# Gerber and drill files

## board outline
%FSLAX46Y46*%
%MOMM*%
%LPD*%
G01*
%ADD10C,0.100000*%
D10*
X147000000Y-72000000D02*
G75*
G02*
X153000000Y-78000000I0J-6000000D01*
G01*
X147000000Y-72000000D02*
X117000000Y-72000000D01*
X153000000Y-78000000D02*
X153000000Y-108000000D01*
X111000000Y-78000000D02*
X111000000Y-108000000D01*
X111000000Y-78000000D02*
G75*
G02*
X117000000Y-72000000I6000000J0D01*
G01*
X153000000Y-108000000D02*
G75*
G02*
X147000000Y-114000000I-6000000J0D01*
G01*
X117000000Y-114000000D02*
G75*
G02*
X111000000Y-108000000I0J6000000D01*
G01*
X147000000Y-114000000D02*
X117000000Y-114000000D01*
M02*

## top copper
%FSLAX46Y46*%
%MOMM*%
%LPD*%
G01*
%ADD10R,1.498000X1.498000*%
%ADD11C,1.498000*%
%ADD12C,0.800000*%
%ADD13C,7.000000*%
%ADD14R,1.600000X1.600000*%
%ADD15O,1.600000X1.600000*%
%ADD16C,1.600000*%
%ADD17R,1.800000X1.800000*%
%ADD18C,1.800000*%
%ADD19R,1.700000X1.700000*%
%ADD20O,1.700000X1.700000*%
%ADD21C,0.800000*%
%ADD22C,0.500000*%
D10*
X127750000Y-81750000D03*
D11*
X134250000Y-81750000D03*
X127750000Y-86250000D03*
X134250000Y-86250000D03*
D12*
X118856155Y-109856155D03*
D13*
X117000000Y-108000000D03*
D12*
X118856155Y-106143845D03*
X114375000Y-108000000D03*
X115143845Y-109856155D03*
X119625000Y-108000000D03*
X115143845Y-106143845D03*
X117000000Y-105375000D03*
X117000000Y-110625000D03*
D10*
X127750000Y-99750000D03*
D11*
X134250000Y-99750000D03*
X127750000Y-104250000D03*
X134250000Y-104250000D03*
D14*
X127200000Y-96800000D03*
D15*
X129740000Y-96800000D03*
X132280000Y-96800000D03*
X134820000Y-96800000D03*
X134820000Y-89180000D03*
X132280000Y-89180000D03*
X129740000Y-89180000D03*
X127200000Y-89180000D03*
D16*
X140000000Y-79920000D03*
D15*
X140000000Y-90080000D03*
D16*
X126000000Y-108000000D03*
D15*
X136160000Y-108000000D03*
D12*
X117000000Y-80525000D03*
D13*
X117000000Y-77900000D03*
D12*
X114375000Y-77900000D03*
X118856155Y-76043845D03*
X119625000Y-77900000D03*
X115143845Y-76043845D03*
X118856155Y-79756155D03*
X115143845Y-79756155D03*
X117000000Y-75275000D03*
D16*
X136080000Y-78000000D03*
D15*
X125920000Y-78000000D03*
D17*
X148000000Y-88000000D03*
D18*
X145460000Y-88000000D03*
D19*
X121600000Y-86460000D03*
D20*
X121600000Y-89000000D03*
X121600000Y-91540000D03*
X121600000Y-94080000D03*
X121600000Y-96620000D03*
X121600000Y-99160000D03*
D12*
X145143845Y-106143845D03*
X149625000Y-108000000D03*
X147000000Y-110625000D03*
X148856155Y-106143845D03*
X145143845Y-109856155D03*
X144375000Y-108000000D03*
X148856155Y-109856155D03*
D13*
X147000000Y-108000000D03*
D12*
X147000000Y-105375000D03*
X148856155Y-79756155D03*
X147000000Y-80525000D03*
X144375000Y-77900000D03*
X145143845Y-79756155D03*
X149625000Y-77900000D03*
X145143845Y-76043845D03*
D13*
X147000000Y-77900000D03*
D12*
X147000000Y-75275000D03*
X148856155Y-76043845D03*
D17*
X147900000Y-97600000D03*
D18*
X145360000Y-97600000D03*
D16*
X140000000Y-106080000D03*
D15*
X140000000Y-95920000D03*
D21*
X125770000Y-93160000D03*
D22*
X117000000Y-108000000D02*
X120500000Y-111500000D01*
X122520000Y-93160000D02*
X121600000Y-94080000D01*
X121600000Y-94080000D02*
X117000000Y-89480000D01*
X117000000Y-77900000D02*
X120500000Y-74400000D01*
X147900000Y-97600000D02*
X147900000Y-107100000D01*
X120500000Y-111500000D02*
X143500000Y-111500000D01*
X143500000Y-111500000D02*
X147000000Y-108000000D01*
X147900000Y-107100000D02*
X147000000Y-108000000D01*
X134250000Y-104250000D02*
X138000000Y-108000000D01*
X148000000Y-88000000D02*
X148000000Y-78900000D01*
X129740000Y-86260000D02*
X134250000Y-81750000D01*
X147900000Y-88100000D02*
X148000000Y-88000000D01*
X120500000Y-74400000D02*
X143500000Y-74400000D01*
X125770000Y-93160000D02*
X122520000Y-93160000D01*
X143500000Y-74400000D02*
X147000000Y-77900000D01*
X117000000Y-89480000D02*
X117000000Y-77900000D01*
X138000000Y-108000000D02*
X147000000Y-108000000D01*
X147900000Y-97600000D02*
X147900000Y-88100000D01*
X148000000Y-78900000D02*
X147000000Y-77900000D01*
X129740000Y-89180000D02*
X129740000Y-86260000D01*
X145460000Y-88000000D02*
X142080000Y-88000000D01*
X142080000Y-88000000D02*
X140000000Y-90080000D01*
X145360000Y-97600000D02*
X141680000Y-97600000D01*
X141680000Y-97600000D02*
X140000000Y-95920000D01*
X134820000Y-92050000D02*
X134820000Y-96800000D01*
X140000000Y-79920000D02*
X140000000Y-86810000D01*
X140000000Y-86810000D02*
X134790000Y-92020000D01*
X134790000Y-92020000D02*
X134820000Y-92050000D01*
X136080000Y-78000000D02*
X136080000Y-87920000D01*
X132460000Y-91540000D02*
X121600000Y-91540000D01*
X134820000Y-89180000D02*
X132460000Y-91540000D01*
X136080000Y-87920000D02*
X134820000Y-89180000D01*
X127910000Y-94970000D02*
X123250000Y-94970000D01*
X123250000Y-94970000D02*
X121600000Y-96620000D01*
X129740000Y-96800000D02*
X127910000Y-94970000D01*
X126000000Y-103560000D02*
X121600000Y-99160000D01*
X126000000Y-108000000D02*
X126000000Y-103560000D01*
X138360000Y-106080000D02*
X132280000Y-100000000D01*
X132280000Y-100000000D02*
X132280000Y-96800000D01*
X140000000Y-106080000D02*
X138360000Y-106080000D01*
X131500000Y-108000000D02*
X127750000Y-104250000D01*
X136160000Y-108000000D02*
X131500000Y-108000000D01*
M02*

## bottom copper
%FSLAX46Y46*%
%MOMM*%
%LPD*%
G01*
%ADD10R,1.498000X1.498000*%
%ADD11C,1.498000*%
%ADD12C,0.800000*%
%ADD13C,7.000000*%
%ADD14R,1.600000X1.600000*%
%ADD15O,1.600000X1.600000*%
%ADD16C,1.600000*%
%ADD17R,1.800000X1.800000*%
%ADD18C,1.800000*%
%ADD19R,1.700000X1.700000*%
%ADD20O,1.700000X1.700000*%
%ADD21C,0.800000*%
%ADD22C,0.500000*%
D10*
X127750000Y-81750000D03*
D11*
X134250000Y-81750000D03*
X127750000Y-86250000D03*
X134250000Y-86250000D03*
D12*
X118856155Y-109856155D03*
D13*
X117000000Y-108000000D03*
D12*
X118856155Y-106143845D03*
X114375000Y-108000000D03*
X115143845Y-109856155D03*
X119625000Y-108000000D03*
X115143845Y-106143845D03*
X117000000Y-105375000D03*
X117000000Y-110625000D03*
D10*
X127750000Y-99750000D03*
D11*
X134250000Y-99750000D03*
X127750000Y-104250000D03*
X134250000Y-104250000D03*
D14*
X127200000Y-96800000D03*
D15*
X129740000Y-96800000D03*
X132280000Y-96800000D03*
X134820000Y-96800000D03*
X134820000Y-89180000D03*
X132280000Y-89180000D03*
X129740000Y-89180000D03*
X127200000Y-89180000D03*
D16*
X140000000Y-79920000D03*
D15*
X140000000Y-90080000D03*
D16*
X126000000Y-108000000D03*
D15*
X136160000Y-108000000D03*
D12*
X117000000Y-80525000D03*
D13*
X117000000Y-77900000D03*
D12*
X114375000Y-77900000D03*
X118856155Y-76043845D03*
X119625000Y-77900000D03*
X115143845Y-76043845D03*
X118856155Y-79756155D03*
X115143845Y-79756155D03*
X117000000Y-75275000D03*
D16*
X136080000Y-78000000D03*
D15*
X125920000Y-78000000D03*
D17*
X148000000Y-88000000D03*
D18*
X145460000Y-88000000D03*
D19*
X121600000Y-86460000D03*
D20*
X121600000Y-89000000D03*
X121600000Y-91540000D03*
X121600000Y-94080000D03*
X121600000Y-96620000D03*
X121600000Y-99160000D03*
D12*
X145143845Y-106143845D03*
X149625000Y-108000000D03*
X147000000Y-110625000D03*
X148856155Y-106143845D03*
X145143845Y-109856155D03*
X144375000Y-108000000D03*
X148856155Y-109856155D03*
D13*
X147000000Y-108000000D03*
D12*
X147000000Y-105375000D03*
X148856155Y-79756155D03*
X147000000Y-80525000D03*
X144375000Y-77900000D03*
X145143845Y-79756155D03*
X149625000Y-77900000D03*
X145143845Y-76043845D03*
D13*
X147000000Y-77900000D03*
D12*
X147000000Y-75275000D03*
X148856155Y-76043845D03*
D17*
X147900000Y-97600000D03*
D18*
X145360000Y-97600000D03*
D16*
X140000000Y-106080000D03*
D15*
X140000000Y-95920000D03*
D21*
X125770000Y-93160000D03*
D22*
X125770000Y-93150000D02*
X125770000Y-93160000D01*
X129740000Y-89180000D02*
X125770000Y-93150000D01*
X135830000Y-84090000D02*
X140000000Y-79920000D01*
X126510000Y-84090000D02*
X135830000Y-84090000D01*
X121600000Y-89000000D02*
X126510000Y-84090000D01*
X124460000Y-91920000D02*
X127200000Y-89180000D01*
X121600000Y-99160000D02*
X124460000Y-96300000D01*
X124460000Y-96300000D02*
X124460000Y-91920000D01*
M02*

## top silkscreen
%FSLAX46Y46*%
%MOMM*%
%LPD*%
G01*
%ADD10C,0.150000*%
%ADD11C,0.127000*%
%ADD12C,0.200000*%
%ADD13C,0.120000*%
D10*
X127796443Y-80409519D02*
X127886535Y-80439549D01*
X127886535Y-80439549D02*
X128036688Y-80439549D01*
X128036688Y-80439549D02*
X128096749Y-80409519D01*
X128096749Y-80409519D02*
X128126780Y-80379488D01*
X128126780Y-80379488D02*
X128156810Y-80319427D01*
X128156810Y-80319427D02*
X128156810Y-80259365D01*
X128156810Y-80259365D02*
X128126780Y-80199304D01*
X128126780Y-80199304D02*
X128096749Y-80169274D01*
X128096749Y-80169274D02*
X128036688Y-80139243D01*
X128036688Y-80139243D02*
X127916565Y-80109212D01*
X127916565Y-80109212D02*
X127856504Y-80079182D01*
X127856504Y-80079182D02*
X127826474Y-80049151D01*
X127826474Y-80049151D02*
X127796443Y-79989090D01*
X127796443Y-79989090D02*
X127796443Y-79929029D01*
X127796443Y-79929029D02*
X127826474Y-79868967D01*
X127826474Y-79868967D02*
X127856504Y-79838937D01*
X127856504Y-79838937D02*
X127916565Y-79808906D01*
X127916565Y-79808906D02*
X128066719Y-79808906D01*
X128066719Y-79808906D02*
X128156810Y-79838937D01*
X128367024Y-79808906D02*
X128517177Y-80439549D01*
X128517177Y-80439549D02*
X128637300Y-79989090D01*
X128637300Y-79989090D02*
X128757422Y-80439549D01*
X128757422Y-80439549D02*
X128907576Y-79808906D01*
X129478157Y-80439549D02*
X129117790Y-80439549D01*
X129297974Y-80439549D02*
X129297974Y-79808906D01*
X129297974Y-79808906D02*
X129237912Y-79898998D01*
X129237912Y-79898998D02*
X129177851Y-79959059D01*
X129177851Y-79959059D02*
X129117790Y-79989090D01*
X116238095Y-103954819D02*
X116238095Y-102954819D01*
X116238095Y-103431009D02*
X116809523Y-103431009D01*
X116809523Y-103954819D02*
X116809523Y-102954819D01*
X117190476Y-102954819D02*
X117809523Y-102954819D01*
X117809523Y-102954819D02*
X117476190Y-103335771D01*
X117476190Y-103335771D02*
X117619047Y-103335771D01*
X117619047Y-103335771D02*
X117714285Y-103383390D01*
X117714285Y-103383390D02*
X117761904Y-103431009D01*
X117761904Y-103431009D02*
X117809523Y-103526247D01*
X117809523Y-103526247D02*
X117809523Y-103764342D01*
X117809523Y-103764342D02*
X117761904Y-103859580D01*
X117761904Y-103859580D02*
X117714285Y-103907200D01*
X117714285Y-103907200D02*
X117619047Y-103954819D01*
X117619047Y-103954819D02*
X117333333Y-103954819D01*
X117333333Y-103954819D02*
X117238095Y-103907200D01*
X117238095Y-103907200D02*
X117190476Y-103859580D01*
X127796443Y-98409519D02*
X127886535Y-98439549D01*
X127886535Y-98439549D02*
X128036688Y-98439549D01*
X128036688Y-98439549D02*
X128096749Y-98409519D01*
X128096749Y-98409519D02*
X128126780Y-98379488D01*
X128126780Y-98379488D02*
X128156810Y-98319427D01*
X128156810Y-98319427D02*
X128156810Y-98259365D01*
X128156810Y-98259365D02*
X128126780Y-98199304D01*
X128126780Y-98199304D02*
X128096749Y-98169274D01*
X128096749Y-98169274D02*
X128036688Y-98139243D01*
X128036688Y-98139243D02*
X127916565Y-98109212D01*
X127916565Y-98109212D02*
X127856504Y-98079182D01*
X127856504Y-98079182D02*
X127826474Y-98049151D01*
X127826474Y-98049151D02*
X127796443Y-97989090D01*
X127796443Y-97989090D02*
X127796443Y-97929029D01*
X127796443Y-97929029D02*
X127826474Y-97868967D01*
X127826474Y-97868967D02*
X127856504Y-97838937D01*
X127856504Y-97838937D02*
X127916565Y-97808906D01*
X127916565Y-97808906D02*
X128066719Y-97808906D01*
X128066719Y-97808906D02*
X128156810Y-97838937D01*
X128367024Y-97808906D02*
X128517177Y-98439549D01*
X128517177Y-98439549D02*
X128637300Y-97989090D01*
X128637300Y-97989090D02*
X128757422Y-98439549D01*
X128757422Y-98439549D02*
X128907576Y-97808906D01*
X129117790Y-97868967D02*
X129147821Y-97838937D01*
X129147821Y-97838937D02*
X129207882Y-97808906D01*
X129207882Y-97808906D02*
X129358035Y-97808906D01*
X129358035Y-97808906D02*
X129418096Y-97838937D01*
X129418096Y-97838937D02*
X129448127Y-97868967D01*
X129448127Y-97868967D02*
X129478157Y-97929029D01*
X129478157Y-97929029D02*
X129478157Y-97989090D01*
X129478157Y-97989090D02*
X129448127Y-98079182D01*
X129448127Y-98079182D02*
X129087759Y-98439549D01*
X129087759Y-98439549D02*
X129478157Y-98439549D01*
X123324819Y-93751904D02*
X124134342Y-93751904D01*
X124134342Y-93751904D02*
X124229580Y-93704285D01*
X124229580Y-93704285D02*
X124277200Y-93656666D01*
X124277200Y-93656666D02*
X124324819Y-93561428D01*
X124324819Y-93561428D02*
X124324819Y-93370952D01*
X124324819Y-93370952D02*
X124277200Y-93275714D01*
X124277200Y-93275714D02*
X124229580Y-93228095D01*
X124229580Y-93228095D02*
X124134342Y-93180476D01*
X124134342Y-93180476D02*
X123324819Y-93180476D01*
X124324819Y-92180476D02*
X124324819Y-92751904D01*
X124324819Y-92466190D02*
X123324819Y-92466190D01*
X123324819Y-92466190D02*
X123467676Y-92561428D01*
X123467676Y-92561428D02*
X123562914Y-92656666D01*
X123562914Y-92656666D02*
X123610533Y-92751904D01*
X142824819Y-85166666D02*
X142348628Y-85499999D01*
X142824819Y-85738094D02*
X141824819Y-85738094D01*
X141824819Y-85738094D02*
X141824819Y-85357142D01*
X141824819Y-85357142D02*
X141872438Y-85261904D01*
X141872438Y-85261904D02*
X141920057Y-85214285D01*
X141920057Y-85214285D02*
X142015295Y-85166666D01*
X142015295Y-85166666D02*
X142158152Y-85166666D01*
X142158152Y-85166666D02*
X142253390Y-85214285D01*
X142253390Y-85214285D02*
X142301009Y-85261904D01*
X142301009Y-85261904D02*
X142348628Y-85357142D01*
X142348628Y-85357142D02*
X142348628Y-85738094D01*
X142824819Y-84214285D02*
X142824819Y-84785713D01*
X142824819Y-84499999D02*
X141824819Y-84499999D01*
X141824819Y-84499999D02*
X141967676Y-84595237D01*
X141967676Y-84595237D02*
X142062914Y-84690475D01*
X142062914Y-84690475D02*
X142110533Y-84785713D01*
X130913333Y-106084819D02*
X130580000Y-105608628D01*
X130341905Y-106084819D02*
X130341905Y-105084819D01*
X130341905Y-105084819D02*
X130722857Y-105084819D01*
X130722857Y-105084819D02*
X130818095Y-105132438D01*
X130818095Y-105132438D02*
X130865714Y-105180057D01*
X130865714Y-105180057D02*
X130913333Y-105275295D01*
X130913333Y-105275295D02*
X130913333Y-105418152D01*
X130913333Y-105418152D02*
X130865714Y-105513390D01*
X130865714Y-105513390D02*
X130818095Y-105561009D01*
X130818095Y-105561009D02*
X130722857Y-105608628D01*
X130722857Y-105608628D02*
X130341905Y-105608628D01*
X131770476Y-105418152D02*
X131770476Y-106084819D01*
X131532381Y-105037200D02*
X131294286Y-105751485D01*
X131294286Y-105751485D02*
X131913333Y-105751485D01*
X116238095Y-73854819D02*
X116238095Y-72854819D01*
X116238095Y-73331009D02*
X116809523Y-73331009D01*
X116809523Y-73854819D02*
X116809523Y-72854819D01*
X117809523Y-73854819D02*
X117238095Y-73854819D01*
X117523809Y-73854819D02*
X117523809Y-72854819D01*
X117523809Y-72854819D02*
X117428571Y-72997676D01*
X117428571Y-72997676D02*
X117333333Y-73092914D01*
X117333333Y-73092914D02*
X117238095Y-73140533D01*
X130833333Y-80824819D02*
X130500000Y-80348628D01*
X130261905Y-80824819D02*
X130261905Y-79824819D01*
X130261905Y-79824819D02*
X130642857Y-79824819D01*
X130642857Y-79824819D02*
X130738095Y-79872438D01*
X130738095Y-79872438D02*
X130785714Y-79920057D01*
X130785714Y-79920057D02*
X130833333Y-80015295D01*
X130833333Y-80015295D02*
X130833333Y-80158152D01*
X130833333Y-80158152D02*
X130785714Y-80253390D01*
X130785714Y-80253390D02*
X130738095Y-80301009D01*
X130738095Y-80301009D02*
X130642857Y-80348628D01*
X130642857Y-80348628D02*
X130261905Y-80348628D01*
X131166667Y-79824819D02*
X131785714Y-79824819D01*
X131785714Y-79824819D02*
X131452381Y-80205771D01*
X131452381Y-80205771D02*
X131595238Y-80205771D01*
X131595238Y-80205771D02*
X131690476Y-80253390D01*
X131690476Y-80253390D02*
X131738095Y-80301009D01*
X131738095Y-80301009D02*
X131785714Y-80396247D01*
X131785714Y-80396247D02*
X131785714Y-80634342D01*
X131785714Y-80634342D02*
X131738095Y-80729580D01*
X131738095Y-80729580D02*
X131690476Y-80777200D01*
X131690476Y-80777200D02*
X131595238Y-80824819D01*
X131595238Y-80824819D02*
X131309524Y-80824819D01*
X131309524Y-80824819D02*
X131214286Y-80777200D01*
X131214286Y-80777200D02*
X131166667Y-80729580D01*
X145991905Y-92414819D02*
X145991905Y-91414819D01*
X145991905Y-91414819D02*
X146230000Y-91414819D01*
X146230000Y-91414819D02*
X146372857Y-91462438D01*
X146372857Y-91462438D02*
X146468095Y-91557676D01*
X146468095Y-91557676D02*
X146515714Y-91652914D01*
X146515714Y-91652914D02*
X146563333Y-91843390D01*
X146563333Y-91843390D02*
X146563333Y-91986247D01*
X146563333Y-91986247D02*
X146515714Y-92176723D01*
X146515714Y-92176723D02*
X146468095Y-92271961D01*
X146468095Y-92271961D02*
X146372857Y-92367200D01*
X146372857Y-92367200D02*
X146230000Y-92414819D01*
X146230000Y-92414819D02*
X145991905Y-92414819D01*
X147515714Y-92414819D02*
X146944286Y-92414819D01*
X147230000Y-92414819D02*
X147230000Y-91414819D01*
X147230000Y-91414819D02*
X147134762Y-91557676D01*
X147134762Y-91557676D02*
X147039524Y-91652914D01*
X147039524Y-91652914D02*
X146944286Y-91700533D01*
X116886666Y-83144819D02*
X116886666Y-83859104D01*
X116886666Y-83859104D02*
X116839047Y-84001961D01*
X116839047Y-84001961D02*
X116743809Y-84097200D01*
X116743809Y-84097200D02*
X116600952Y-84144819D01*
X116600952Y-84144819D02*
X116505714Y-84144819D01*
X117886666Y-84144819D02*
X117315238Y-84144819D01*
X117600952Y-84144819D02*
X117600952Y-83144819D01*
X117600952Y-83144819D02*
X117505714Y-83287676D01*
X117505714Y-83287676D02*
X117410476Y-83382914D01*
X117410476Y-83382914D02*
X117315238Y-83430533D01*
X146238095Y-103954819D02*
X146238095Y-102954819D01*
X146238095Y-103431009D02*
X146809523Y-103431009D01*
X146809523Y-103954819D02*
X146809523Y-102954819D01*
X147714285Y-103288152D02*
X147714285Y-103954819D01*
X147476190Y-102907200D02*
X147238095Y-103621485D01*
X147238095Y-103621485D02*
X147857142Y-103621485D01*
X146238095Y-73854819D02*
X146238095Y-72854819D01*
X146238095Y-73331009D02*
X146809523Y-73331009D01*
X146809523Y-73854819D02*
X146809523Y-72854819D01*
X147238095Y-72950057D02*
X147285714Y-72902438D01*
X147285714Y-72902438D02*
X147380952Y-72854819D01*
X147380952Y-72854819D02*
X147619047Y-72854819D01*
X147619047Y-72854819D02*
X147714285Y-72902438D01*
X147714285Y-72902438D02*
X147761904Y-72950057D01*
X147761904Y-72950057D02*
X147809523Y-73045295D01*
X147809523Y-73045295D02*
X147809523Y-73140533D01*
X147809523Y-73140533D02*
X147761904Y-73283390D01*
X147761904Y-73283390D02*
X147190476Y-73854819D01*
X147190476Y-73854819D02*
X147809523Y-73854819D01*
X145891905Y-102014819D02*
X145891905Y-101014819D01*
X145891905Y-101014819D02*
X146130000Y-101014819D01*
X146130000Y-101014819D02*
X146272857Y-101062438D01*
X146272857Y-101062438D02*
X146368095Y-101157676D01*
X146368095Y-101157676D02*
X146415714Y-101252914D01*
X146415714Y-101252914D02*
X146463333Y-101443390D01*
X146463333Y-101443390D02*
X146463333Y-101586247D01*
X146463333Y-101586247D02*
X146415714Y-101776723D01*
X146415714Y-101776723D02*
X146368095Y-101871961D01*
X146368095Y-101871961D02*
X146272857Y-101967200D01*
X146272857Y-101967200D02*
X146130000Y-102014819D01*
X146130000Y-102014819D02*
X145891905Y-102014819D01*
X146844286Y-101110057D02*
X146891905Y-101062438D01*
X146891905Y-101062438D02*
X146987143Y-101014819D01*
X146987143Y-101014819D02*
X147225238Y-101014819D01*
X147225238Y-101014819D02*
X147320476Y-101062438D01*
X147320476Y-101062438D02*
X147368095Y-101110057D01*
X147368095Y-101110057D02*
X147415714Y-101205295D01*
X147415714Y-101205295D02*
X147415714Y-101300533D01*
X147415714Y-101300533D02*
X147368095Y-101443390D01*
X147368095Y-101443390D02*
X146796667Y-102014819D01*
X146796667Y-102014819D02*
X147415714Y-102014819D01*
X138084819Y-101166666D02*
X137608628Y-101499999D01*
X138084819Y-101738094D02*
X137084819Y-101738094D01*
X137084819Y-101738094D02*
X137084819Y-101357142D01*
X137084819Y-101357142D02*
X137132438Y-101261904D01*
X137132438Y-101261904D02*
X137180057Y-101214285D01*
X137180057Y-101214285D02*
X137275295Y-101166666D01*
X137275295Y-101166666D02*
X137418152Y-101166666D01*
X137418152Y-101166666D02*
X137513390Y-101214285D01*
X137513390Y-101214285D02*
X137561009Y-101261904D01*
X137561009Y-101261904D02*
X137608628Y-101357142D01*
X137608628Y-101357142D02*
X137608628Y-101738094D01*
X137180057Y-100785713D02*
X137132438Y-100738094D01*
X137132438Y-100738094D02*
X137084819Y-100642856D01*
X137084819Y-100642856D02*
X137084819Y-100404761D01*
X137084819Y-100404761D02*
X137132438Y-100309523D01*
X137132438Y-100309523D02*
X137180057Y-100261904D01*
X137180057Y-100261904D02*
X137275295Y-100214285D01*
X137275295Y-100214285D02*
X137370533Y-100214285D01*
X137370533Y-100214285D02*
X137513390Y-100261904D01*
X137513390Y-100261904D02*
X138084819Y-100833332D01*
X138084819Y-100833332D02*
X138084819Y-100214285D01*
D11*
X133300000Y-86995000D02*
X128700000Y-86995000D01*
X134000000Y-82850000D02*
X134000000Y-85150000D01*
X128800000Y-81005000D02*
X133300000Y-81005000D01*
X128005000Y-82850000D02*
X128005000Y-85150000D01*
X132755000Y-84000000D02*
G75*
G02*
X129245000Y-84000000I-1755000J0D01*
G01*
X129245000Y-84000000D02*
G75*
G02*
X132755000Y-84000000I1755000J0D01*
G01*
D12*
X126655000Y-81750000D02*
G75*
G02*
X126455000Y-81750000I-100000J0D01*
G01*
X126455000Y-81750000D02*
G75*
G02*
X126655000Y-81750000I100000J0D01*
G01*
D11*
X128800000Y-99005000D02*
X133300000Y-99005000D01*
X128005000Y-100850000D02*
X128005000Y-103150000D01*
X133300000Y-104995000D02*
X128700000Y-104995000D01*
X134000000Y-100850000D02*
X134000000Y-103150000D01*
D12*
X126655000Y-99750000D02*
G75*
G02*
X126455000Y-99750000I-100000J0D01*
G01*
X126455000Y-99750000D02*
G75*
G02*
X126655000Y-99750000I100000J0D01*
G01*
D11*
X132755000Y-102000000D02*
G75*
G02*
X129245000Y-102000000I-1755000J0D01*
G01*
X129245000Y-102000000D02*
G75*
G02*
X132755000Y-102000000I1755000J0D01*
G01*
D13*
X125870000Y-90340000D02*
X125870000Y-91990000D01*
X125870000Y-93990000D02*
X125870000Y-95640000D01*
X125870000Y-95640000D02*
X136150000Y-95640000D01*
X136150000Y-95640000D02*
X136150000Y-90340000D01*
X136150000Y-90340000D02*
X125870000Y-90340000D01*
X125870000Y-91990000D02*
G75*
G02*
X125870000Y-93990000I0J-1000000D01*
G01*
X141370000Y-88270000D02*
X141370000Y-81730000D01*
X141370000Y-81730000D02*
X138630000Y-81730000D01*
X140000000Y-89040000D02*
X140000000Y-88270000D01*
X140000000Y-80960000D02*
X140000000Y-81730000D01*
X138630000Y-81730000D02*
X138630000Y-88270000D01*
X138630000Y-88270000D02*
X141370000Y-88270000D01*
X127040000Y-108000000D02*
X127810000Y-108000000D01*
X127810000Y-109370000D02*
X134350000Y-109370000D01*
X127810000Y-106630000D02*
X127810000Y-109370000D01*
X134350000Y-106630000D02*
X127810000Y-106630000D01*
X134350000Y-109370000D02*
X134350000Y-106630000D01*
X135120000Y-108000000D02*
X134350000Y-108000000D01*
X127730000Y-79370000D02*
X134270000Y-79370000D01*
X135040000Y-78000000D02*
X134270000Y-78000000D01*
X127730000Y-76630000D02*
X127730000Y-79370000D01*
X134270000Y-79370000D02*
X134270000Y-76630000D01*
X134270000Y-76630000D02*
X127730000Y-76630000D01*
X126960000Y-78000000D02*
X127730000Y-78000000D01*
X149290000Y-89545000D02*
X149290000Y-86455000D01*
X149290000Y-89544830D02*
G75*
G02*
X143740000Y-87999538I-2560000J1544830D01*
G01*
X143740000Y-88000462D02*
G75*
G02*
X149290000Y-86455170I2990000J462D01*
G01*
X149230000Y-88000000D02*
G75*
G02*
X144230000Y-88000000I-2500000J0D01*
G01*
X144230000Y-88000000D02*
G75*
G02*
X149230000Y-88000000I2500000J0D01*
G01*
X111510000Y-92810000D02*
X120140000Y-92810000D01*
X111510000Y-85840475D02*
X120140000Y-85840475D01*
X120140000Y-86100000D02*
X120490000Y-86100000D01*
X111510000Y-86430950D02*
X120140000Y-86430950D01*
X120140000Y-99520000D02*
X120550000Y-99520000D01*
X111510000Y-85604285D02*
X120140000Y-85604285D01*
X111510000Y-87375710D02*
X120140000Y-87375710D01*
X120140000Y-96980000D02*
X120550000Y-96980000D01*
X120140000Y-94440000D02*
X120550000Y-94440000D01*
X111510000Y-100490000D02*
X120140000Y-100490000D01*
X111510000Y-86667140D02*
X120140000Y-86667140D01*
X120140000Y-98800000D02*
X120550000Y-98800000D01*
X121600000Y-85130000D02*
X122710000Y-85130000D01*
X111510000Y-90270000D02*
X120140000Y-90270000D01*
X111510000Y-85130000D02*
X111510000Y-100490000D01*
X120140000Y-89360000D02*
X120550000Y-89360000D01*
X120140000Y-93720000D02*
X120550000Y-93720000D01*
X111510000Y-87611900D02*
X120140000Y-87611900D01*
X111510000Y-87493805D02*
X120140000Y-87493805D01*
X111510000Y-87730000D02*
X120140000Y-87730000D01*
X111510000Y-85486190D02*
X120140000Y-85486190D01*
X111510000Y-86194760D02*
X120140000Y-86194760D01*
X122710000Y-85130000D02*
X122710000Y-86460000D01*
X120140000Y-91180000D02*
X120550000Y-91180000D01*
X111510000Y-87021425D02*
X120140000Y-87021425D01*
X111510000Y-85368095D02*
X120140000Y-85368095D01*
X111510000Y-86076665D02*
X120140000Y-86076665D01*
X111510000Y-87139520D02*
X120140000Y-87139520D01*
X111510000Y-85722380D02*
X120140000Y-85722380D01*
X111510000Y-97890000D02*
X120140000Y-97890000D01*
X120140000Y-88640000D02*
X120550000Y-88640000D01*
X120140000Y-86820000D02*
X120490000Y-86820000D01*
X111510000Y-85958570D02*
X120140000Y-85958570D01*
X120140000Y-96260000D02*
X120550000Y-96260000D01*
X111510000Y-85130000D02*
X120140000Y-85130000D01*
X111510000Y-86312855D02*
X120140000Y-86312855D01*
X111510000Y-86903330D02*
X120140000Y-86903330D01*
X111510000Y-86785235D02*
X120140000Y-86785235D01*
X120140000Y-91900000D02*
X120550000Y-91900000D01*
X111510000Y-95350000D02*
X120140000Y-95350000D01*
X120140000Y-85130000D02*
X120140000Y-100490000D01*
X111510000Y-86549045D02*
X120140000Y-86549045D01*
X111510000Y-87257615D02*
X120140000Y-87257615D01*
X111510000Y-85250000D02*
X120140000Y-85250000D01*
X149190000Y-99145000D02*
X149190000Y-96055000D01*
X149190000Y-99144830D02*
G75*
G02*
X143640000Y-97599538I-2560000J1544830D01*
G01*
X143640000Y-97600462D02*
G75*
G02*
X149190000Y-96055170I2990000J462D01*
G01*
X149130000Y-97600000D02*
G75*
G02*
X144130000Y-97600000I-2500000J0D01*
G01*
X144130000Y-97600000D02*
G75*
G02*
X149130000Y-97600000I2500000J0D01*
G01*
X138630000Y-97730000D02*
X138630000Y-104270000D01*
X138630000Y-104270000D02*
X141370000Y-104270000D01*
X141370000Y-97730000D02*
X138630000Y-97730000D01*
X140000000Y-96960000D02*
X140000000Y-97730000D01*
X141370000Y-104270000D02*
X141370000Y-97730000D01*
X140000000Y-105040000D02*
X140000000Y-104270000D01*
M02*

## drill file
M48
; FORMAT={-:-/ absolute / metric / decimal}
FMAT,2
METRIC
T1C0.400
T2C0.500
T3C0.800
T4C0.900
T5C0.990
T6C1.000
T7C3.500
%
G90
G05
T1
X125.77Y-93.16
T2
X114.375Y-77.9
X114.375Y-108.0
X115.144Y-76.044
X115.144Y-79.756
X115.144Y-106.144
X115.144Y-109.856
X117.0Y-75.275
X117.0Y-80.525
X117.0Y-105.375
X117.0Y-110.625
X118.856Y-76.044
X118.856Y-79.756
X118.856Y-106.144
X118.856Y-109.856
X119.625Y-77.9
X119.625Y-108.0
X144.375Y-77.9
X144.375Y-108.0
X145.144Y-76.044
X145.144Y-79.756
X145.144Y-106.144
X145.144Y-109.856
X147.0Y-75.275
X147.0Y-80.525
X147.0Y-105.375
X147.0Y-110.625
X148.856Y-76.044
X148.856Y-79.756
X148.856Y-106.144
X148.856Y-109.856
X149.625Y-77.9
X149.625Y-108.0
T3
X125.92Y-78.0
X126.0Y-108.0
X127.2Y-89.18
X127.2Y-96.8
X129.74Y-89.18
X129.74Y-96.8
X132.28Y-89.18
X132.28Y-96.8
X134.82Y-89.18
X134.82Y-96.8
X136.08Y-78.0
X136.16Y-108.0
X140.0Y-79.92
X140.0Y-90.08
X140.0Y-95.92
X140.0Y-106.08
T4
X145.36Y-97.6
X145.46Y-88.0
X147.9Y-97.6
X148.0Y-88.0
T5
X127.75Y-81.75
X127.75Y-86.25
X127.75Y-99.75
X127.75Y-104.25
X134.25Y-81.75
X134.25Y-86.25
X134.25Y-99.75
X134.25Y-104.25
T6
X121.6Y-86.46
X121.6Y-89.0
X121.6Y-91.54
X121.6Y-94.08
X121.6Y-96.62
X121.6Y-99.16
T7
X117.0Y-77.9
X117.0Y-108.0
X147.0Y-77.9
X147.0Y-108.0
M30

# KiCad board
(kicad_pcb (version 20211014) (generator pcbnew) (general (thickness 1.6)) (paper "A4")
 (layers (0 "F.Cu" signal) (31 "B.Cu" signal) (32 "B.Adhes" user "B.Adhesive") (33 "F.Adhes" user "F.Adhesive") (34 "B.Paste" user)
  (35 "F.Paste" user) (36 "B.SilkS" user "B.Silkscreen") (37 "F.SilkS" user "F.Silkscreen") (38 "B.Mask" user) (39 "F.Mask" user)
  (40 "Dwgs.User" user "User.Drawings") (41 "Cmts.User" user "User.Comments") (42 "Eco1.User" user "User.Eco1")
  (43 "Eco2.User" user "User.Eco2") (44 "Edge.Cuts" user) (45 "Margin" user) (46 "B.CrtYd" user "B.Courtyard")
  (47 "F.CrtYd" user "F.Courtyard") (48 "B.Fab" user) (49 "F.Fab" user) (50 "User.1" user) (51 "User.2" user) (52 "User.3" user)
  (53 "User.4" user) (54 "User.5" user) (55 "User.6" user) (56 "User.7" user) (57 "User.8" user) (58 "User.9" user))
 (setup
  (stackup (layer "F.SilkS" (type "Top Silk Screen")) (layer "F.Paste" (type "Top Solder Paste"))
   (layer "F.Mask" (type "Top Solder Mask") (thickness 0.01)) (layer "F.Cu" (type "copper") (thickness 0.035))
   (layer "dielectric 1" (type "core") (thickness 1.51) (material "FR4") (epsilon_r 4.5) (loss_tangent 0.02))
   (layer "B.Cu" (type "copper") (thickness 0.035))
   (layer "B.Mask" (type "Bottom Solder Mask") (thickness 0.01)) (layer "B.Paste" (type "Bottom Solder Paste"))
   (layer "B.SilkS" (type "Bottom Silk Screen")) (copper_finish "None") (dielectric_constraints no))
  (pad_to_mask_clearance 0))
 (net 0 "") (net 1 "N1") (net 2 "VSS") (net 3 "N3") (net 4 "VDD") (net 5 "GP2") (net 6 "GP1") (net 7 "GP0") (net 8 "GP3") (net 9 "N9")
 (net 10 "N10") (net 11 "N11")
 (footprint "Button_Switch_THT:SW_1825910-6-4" (layer "F.Cu") (at 131 84)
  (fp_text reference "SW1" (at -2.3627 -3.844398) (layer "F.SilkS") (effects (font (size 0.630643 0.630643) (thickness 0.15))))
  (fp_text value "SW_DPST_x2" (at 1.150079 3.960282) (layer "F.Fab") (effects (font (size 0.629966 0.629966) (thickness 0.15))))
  (fp_line (start 2.3 2.995) (end -2.3 2.995) (layer "F.SilkS") (width 0.127))
  (fp_line (start 3 -1.15) (end 3 1.15) (layer "F.SilkS") (width 0.127))
  (fp_line (start -2.2 -2.995) (end 2.3 -2.995) (layer "F.SilkS") (width 0.127))
  (fp_line (start -2.995 -1.15) (end -2.995 1.15) (layer "F.SilkS") (width 0.127))
  (fp_circle (center 0 0) (end 1.755 0) (layer "F.SilkS") (width 0.127) (fill none))
  (fp_circle (center -4.445 -2.25) (end -4.345 -2.25) (layer "F.SilkS") (width 0.2) (fill none))
  (pad "1" thru_hole rect locked (at -3.25 -2.25) (size 1.498 1.498) (drill 0.99) (layers *.Cu *.Mask) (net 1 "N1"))
  (pad "2" thru_hole circle locked (at 3.25 -2.25) (size 1.498 1.498) (drill 0.99) (layers *.Cu *.Mask) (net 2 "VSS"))
  (pad "3" thru_hole circle locked (at -3.25 2.25) (size 1.498 1.498) (drill 0.99) (layers *.Cu *.Mask))
  (pad "4" thru_hole circle locked (at 3.25 2.25) (size 1.498 1.498) (drill 0.99) (layers *.Cu *.Mask)))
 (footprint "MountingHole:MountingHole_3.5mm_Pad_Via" (layer "F.Cu") (at 117 108)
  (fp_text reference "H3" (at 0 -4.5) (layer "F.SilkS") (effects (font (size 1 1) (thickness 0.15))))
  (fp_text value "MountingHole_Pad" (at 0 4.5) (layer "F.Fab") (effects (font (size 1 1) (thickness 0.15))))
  (pad "1" thru_hole circle (at 1.856155 1.856155) (size 0.8 0.8) (drill 0.5) (layers *.Cu *.Mask) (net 2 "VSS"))
  (pad "1" thru_hole circle (at 0 0) (size 7 7) (drill 3.5) (layers *.Cu *.Mask) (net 2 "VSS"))
  (pad "1" thru_hole circle (at 1.856155 -1.856155) (size 0.8 0.8) (drill 0.5) (layers *.Cu *.Mask) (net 2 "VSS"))
  (pad "1" thru_hole circle (at -2.625 0) (size 0.8 0.8) (drill 0.5) (layers *.Cu *.Mask) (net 2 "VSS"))
  (pad "1" thru_hole circle (at -1.856155 1.856155) (size 0.8 0.8) (drill 0.5) (layers *.Cu *.Mask) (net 2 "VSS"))
  (pad "1" thru_hole circle (at 2.625 0) (size 0.8 0.8) (drill 0.5) (layers *.Cu *.Mask) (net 2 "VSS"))
  (pad "1" thru_hole circle (at -1.856155 -1.856155) (size 0.8 0.8) (drill 0.5) (layers *.Cu *.Mask) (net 2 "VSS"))
  (pad "1" thru_hole circle (at 0 -2.625) (size 0.8 0.8) (drill 0.5) (layers *.Cu *.Mask) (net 2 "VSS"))
  (pad "1" thru_hole circle (at 0 2.625) (size 0.8 0.8) (drill 0.5) (layers *.Cu *.Mask) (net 2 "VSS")))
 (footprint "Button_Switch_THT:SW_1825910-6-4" (layer "F.Cu") (at 131 102)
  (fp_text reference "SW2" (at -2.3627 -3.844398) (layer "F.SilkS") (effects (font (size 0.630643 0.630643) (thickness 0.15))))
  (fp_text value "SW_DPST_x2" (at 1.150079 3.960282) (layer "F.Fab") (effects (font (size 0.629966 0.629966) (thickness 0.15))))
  (fp_line (start -2.2 -2.995) (end 2.3 -2.995) (layer "F.SilkS") (width 0.127))
  (fp_line (start -2.995 -1.15) (end -2.995 1.15) (layer "F.SilkS") (width 0.127))
  (fp_line (start 2.3 2.995) (end -2.3 2.995) (layer "F.SilkS") (width 0.127))
  (fp_line (start 3 -1.15) (end 3 1.15) (layer "F.SilkS") (width 0.127))
  (fp_circle (center -4.445 -2.25) (end -4.345 -2.25) (layer "F.SilkS") (width 0.2) (fill none))
  (fp_circle (center 0 0) (end 1.755 0) (layer "F.SilkS") (width 0.127) (fill none))
  (pad "1" thru_hole rect locked (at -3.25 -2.25) (size 1.498 1.498) (drill 0.99) (layers *.Cu *.Mask))
  (pad "2" thru_hole circle locked (at 3.25 -2.25) (size 1.498 1.498) (drill 0.99) (layers *.Cu *.Mask))
  (pad "3" thru_hole circle locked (at -3.25 2.25) (size 1.498 1.498) (drill 0.99) (layers *.Cu *.Mask) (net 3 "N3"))
  (pad "4" thru_hole circle locked (at 3.25 2.25) (size 1.498 1.498) (drill 0.99) (layers *.Cu *.Mask) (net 2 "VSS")))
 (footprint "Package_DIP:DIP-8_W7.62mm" (layer "F.Cu") (at 127.2 96.8 90)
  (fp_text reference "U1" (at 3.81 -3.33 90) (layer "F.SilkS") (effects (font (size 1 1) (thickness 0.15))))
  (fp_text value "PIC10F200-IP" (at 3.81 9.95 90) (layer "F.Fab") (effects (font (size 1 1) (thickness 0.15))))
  (fp_line (start 6.46 -1.33) (end 4.81 -1.33) (layer "F.SilkS") (width 0.12))
  (fp_line (start 2.81 -1.33) (end 1.16 -1.33) (layer "F.SilkS") (width 0.12))
  (fp_line (start 1.16 -1.33) (end 1.16 8.95) (layer "F.SilkS") (width 0.12))
  (fp_line (start 1.16 8.95) (end 6.46 8.95) (layer "F.SilkS") (width 0.12))
  (fp_line (start 6.46 8.95) (end 6.46 -1.33) (layer "F.SilkS") (width 0.12))
  (fp_arc (start 4.81 -1.33) (mid 3.81 -0.33) (end 2.81 -1.33) (layer "F.SilkS") (width 0.12))
  (pad "1" thru_hole rect (at 0 0 90) (size 1.6 1.6) (drill 0.8) (layers *.Cu *.Mask))
  (pad "2" thru_hole oval (at 0 2.54 90) (size 1.6 1.6) (drill 0.8) (layers *.Cu *.Mask) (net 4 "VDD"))
  (pad "3" thru_hole oval (at 0 5.08 90) (size 1.6 1.6) (drill 0.8) (layers *.Cu *.Mask) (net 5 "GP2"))
  (pad "4" thru_hole oval (at 0 7.62 90) (size 1.6 1.6) (drill 0.8) (layers *.Cu *.Mask) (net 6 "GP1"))
  (pad "5" thru_hole oval (at 7.62 7.62 90) (size 1.6 1.6) (drill 0.8) (layers *.Cu *.Mask) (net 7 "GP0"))
  (pad "6" thru_hole oval (at 7.62 5.08 90) (size 1.6 1.6) (drill 0.8) (layers *.Cu *.Mask))
  (pad "7" thru_hole oval (at 7.62 2.54 90) (size 1.6 1.6) (drill 0.8) (layers *.Cu *.Mask) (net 2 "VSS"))
  (pad "8" thru_hole oval (at 7.62 0 90) (size 1.6 1.6) (drill 0.8) (layers *.Cu *.Mask) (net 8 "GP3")))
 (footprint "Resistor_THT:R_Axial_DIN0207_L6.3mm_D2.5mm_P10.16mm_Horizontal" (layer "F.Cu") (at 140 79.92 -90)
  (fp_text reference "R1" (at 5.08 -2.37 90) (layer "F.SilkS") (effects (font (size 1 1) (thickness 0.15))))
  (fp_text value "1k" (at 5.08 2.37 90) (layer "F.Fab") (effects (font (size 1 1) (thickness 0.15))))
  (fp_line (start 8.35 -1.37) (end 1.81 -1.37) (layer "F.SilkS") (width 0.12))
  (fp_line (start 1.81 -1.37) (end 1.81 1.37) (layer "F.SilkS") (width 0.12))
  (fp_line (start 9.12 0) (end 8.35 0) (layer "F.SilkS") (width 0.12))
  (fp_line (start 1.04 0) (end 1.81 0) (layer "F.SilkS") (width 0.12))
  (fp_line (start 1.81 1.37) (end 8.35 1.37) (layer "F.SilkS") (width 0.12))
  (fp_line (start 8.35 1.37) (end 8.35 -1.37) (layer "F.SilkS") (width 0.12))
  (pad "1" thru_hole circle (at 0 0 270) (size 1.6 1.6) (drill 0.8) (layers *.Cu *.Mask) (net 6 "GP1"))
  (pad "2" thru_hole oval (at 10.16 0 270) (size 1.6 1.6) (drill 0.8) (layers *.Cu *.Mask) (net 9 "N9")))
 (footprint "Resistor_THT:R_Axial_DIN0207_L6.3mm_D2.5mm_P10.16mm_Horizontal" (layer "F.Cu") (at 126 108)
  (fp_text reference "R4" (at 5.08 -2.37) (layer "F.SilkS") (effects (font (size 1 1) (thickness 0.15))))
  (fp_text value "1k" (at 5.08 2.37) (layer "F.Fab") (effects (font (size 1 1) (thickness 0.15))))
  (fp_line (start 1.04 0) (end 1.81 0) (layer "F.SilkS") (width 0.12))
  (fp_line (start 1.81 1.37) (end 8.35 1.37) (layer "F.SilkS") (width 0.12))
  (fp_line (start 1.81 -1.37) (end 1.81 1.37) (layer "F.SilkS") (width 0.12))
  (fp_line (start 8.35 -1.37) (end 1.81 -1.37) (layer "F.SilkS") (width 0.12))
  (fp_line (start 8.35 1.37) (end 8.35 -1.37) (layer "F.SilkS") (width 0.12))
  (fp_line (start 9.12 0) (end 8.35 0) (layer "F.SilkS") (width 0.12))
  (pad "1" thru_hole circle (at 0 0) (size 1.6 1.6) (drill 0.8) (layers *.Cu *.Mask) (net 8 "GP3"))
  (pad "2" thru_hole oval (at 10.16 0) (size 1.6 1.6) (drill 0.8) (layers *.Cu *.Mask) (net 3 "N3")))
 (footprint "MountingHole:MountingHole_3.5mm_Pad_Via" (layer "F.Cu") (at 117 77.9)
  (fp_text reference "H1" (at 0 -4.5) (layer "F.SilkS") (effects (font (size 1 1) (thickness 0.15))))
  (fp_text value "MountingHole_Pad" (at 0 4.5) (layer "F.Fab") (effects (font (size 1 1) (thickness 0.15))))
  (pad "1" thru_hole circle (at 0 2.625) (size 0.8 0.8) (drill 0.5) (layers *.Cu *.Mask) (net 2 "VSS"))
  (pad "1" thru_hole circle (at 0 0) (size 7 7) (drill 3.5) (layers *.Cu *.Mask) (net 2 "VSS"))
  (pad "1" thru_hole circle (at -2.625 0) (size 0.8 0.8) (drill 0.5) (layers *.Cu *.Mask) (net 2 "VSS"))
  (pad "1" thru_hole circle (at 1.856155 -1.856155) (size 0.8 0.8) (drill 0.5) (layers *.Cu *.Mask) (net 2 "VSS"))
  (pad "1" thru_hole circle (at 2.625 0) (size 0.8 0.8) (drill 0.5) (layers *.Cu *.Mask) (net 2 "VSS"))
  (pad "1" thru_hole circle (at -1.856155 -1.856155) (size 0.8 0.8) (drill 0.5) (layers *.Cu *.Mask) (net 2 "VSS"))
  (pad "1" thru_hole circle (at 1.856155 1.856155) (size 0.8 0.8) (drill 0.5) (layers *.Cu *.Mask) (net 2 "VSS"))
  (pad "1" thru_hole circle (at -1.856155 1.856155) (size 0.8 0.8) (drill 0.5) (layers *.Cu *.Mask) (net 2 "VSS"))
  (pad "1" thru_hole circle (at 0 -2.625) (size 0.8 0.8) (drill 0.5) (layers *.Cu *.Mask) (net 2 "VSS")))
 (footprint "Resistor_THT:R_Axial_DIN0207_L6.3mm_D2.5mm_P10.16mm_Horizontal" (layer "F.Cu") (at 136.08 78 180)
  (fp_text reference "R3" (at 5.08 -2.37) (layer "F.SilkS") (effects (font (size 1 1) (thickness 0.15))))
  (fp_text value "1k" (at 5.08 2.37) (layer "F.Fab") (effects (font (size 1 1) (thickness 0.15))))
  (fp_line (start 8.35 -1.37) (end 1.81 -1.37) (layer "F.SilkS") (width 0.12))
  (fp_line (start 1.04 0) (end 1.81 0) (layer "F.SilkS") (width 0.12))
  (fp_line (start 8.35 1.37) (end 8.35 -1.37) (layer "F.SilkS") (width 0.12))
  (fp_line (start 1.81 -1.37) (end 1.81 1.37) (layer "F.SilkS") (width 0.12))
  (fp_line (start 1.81 1.37) (end 8.35 1.37) (layer "F.SilkS") (width 0.12))
  (fp_line (start 9.12 0) (end 8.35 0) (layer "F.SilkS") (width 0.12))
  (pad "1" thru_hole circle (at 0 0 180) (size 1.6 1.6) (drill 0.8) (layers *.Cu *.Mask) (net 7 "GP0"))
  (pad "2" thru_hole oval (at 10.16 0 180) (size 1.6 1.6) (drill 0.8) (layers *.Cu *.Mask) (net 1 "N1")))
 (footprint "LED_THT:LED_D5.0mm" (layer "F.Cu") (at 148 88 180)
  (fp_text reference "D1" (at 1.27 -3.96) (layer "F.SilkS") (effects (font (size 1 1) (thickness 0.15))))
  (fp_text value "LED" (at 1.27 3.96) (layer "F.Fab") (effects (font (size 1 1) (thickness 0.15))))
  (fp_line (start -1.29 -1.545) (end -1.29 1.545) (layer "F.SilkS") (width 0.12))
  (fp_arc (start -1.29 -1.54483) (mid 2.072002 -2.880433) (end 4.26 0.000462) (layer "F.SilkS") (width 0.12))
  (fp_arc (start 4.26 -0.000462) (mid 2.072002 2.880433) (end -1.29 1.54483) (layer "F.SilkS") (width 0.12))
  (fp_circle (center 1.27 0) (end 3.77 0) (layer "F.SilkS") (width 0.12) (fill none))
  (pad "1" thru_hole rect (at 0 0 180) (size 1.8 1.8) (drill 0.9) (layers *.Cu *.Mask) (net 2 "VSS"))
  (pad "2" thru_hole circle (at 2.54 0 180) (size 1.8 1.8) (drill 0.9) (layers *.Cu *.Mask) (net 9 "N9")))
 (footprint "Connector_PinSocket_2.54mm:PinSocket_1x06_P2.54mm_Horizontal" (layer "F.Cu") (at 121.6 86.46)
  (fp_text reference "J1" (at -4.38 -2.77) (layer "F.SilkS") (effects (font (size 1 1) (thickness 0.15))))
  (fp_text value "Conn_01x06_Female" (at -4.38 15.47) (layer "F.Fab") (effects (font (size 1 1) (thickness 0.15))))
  (fp_line (start -10.09 6.35) (end -1.46 6.35) (layer "F.SilkS") (width 0.12))
  (fp_line (start -10.09 -0.619525) (end -1.46 -0.619525) (layer "F.SilkS") (width 0.12))
  (fp_line (start -1.46 -0.36) (end -1.11 -0.36) (layer "F.SilkS") (width 0.12))
  (fp_line (start -10.09 -0.02905) (end -1.46 -0.02905) (layer "F.SilkS") (width 0.12))
  (fp_line (start -1.46 13.06) (end -1.05 13.06) (layer "F.SilkS") (width 0.12))
  (fp_line (start -10.09 -0.855715) (end -1.46 -0.855715) (layer "F.SilkS") (width 0.12))
  (fp_line (start -10.09 0.91571) (end -1.46 0.91571) (layer "F.SilkS") (width 0.12))
  (fp_line (start -1.46 10.52) (end -1.05 10.52) (layer "F.SilkS") (width 0.12))
  (fp_line (start -1.46 7.98) (end -1.05 7.98) (layer "F.SilkS") (width 0.12))
  (fp_line (start -10.09 14.03) (end -1.46 14.03) (layer "F.SilkS") (width 0.12))
  (fp_line (start -10.09 0.20714) (end -1.46 0.20714) (layer "F.SilkS") (width 0.12))
  (fp_line (start -1.46 12.34) (end -1.05 12.34) (layer "F.SilkS") (width 0.12))
  (fp_line (start 0 -1.33) (end 1.11 -1.33) (layer "F.SilkS") (width 0.12))
  (fp_line (start -10.09 3.81) (end -1.46 3.81) (layer "F.SilkS") (width 0.12))
  (fp_line (start -10.09 -1.33) (end -10.09 14.03) (layer "F.SilkS") (width 0.12))
  (fp_line (start -1.46 2.9) (end -1.05 2.9) (layer "F.SilkS") (width 0.12))
  (fp_line (start -1.46 7.26) (end -1.05 7.26) (layer "F.SilkS") (width 0.12))
  (fp_line (start -10.09 1.1519) (end -1.46 1.1519) (layer "F.SilkS") (width 0.12))
  (fp_line (start -10.09 1.033805) (end -1.46 1.033805) (layer "F.SilkS") (width 0.12))
  (fp_line (start -10.09 1.27) (end -1.46 1.27) (layer "F.SilkS") (width 0.12))
  (fp_line (start -10.09 -0.97381) (end -1.46 -0.97381) (layer "F.SilkS") (width 0.12))
  (fp_line (start -10.09 -0.26524) (end -1.46 -0.26524) (layer "F.SilkS") (width 0.12))
  (fp_line (start 1.11 -1.33) (end 1.11 0) (layer "F.SilkS") (width 0.12))
  (fp_line (start -1.46 4.72) (end -1.05 4.72) (layer "F.SilkS") (width 0.12))
  (fp_line (start -10.09 0.561425) (end -1.46 0.561425) (layer "F.SilkS") (width 0.12))
  (fp_line (start -10.09 -1.091905) (end -1.46 -1.091905) (layer "F.SilkS") (width 0.12))
  (fp_line (start -10.09 -0.383335) (end -1.46 -0.383335) (layer "F.SilkS") (width 0.12))
  (fp_line (start -10.09 0.67952) (end -1.46 0.67952) (layer "F.SilkS") (width 0.12))
  (fp_line (start -10.09 -0.73762) (end -1.46 -0.73762) (layer "F.SilkS") (width 0.12))
  (fp_line (start -10.09 11.43) (end -1.46 11.43) (layer "F.SilkS") (width 0.12))
  (fp_line (start -1.46 2.18) (end -1.05 2.18) (layer "F.SilkS") (width 0.12))
  (fp_line (start -1.46 0.36) (end -1.11 0.36) (layer "F.SilkS") (width 0.12))
  (fp_line (start -10.09 -0.50143) (end -1.46 -0.50143) (layer "F.SilkS") (width 0.12))
  (fp_line (start -1.46 9.8) (end -1.05 9.8) (layer "F.SilkS") (width 0.12))
  (fp_line (start -10.09 -1.33) (end -1.46 -1.33) (layer "F.SilkS") (width 0.12))
  (fp_line (start -10.09 -0.147145) (end -1.46 -0.147145) (layer "F.SilkS") (width 0.12))
  (fp_line (start -10.09 0.44333) (end -1.46 0.44333) (layer "F.SilkS") (width 0.12))
  (fp_line (start -10.09 0.325235) (end -1.46 0.325235) (layer "F.SilkS") (width 0.12))
  (fp_line (start -1.46 5.44) (end -1.05 5.44) (layer "F.SilkS") (width 0.12))
  (fp_line (start -10.09 8.89) (end -1.46 8.89) (layer "F.SilkS") (width 0.12))
  (fp_line (start -1.46 -1.33) (end -1.46 14.03) (layer "F.SilkS") (width 0.12))
  (fp_line (start -10.09 0.089045) (end -1.46 0.089045) (layer "F.SilkS") (width 0.12))
  (fp_line (start -10.09 0.797615) (end -1.46 0.797615) (layer "F.SilkS") (width 0.12))
  (fp_line (start -10.09 -1.21) (end -1.46 -1.21) (layer "F.SilkS") (width 0.12))
  (pad "1" thru_hole rect (at 0 0) (size 1.7 1.7) (drill 1) (layers *.Cu *.Mask) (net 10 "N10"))
  (pad "2" thru_hole oval (at 0 2.54) (size 1.7 1.7) (drill 1) (layers *.Cu *.Mask) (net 6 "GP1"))
  (pad "3" thru_hole oval (at 0 5.08) (size 1.7 1.7) (drill 1) (layers *.Cu *.Mask) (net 7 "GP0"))
  (pad "4" thru_hole oval (at 0 7.62) (size 1.7 1.7) (drill 1) (layers *.Cu *.Mask) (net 2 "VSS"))
  (pad "5" thru_hole oval (at 0 10.16) (size 1.7 1.7) (drill 1) (layers *.Cu *.Mask) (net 4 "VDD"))
  (pad "6" thru_hole oval (at 0 12.7) (size 1.7 1.7) (drill 1) (layers *.Cu *.Mask) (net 8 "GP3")))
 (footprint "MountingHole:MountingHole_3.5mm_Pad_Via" (layer "F.Cu") (at 147 108)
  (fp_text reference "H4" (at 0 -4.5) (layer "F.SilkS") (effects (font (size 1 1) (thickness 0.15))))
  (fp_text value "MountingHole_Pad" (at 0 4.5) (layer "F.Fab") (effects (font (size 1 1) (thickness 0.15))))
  (pad "1" thru_hole circle (at -1.856155 -1.856155) (size 0.8 0.8) (drill 0.5) (layers *.Cu *.Mask) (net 2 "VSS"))
  (pad "1" thru_hole circle (at 2.625 0) (size 0.8 0.8) (drill 0.5) (layers *.Cu *.Mask) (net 2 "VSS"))
  (pad "1" thru_hole circle (at 0 2.625) (size 0.8 0.8) (drill 0.5) (layers *.Cu *.Mask) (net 2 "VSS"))
  (pad "1" thru_hole circle (at 1.856155 -1.856155) (size 0.8 0.8) (drill 0.5) (layers *.Cu *.Mask) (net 2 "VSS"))
  (pad "1" thru_hole circle (at -1.856155 1.856155) (size 0.8 0.8) (drill 0.5) (layers *.Cu *.Mask) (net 2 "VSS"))
  (pad "1" thru_hole circle (at -2.625 0) (size 0.8 0.8) (drill 0.5) (layers *.Cu *.Mask) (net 2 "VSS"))
  (pad "1" thru_hole circle (at 1.856155 1.856155) (size 0.8 0.8) (drill 0.5) (layers *.Cu *.Mask) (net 2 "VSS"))
  (pad "1" thru_hole circle (at 0 0) (size 7 7) (drill 3.5) (layers *.Cu *.Mask) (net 2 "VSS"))
  (pad "1" thru_hole circle (at 0 -2.625) (size 0.8 0.8) (drill 0.5) (layers *.Cu *.Mask) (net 2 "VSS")))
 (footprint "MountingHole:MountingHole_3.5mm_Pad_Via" (layer "F.Cu") (at 147 77.9)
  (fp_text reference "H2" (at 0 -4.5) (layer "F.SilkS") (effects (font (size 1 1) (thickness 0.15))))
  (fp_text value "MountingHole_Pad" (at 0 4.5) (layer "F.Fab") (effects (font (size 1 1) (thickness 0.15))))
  (pad "1" thru_hole circle (at 1.856155 1.856155) (size 0.8 0.8) (drill 0.5) (layers *.Cu *.Mask) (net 2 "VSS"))
  (pad "1" thru_hole circle (at 0 2.625) (size 0.8 0.8) (drill 0.5) (layers *.Cu *.Mask) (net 2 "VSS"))
  (pad "1" thru_hole circle (at -2.625 0) (size 0.8 0.8) (drill 0.5) (layers *.Cu *.Mask) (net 2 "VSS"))
  (pad "1" thru_hole circle (at -1.856155 1.856155) (size 0.8 0.8) (drill 0.5) (layers *.Cu *.Mask) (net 2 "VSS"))
  (pad "1" thru_hole circle (at 2.625 0) (size 0.8 0.8) (drill 0.5) (layers *.Cu *.Mask) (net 2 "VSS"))
  (pad "1" thru_hole circle (at -1.856155 -1.856155) (size 0.8 0.8) (drill 0.5) (layers *.Cu *.Mask) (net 2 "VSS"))
  (pad "1" thru_hole circle (at 0 0) (size 7 7) (drill 3.5) (layers *.Cu *.Mask) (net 2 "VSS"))
  (pad "1" thru_hole circle (at 0 -2.625) (size 0.8 0.8) (drill 0.5) (layers *.Cu *.Mask) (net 2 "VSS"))
  (pad "1" thru_hole circle (at 1.856155 -1.856155) (size 0.8 0.8) (drill 0.5) (layers *.Cu *.Mask) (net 2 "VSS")))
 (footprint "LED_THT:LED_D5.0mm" (layer "F.Cu") (at 147.9 97.6 180)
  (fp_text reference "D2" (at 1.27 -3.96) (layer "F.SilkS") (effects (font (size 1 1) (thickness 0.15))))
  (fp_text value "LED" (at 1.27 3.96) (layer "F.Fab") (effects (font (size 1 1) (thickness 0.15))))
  (fp_line (start -1.29 -1.545) (end -1.29 1.545) (layer "F.SilkS") (width 0.12))
  (fp_arc (start -1.29 -1.54483) (mid 2.072002 -2.880433) (end 4.26 0.000462) (layer "F.SilkS") (width 0.12))
  (fp_arc (start 4.26 -0.000462) (mid 2.072002 2.880433) (end -1.29 1.54483) (layer "F.SilkS") (width 0.12))
  (fp_circle (center 1.27 0) (end 3.77 0) (layer "F.SilkS") (width 0.12) (fill none))
  (pad "1" thru_hole rect (at 0 0 180) (size 1.8 1.8) (drill 0.9) (layers *.Cu *.Mask) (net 2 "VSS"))
  (pad "2" thru_hole circle (at 2.54 0 180) (size 1.8 1.8) (drill 0.9) (layers *.Cu *.Mask) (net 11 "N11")))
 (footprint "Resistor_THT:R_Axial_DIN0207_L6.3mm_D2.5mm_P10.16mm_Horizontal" (layer "F.Cu") (at 140 106.08 90)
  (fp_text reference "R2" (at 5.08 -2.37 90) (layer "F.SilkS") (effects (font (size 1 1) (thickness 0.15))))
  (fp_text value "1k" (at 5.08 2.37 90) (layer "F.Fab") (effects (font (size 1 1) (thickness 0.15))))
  (fp_line (start 8.35 -1.37) (end 1.81 -1.37) (layer "F.SilkS") (width 0.12))
  (fp_line (start 1.81 -1.37) (end 1.81 1.37) (layer "F.SilkS") (width 0.12))
  (fp_line (start 8.35 1.37) (end 8.35 -1.37) (layer "F.SilkS") (width 0.12))
  (fp_line (start 9.12 0) (end 8.35 0) (layer "F.SilkS") (width 0.12))
  (fp_line (start 1.81 1.37) (end 8.35 1.37) (layer "F.SilkS") (width 0.12))
  (fp_line (start 1.04 0) (end 1.81 0) (layer "F.SilkS") (width 0.12))
  (pad "1" thru_hole circle (at 0 0 90) (size 1.6 1.6) (drill 0.8) (layers *.Cu *.Mask) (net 5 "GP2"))
  (pad "2" thru_hole oval (at 10.16 0 90) (size 1.6 1.6) (drill 0.8) (layers *.Cu *.Mask) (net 11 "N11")))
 (gr_arc (start 147 72) (mid 151.242641 73.757359) (end 153 78) (layer "Edge.Cuts") (width 0.1))
 (gr_line (start 147 72) (end 117 72) (layer "Edge.Cuts") (width 0.1))
 (gr_line (start 153 78) (end 153 108) (layer "Edge.Cuts") (width 0.1))
 (gr_line (start 111 78) (end 111 108) (layer "Edge.Cuts") (width 0.1))
 (gr_arc (start 111 78) (mid 112.757359 73.757359) (end 117 72) (layer "Edge.Cuts") (width 0.1))
 (gr_arc (start 153 108) (mid 151.242641 112.242641) (end 147 114) (layer "Edge.Cuts") (width 0.1))
 (gr_arc (start 117 114) (mid 112.757359 112.242641) (end 111 108) (layer "Edge.Cuts") (width 0.1))
 (gr_line (start 147 114) (end 117 114) (layer "Edge.Cuts") (width 0.1))
 (segment (start 117 108) (end 120.5 111.5) (width 0.5) (layer "F.Cu") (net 2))
 (segment (start 122.52 93.16) (end 121.6 94.08) (width 0.5) (layer "F.Cu") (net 2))
 (segment (start 121.6 94.08) (end 117 89.48) (width 0.5) (layer "F.Cu") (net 2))
 (segment (start 117 77.9) (end 120.5 74.4) (width 0.5) (layer "F.Cu") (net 2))
 (segment (start 147.9 97.6) (end 147.9 107.1) (width 0.5) (layer "F.Cu") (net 2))
 (segment (start 120.5 111.5) (end 143.5 111.5) (width 0.5) (layer "F.Cu") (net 2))
 (segment (start 143.5 111.5) (end 147 108) (width 0.5) (layer "F.Cu") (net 2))
 (segment (start 147.9 107.1) (end 147 108) (width 0.5) (layer "F.Cu") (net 2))
 (segment (start 134.25 104.25) (end 138 108) (width 0.5) (layer "F.Cu") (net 2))
 (segment (start 148 88) (end 148 78.9) (width 0.5) (layer "F.Cu") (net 2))
 (segment (start 129.74 86.26) (end 134.25 81.75) (width 0.5) (layer "F.Cu") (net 2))
 (segment (start 147.9 88.1) (end 148 88) (width 0.5) (layer "F.Cu") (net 2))
 (segment (start 120.5 74.4) (end 143.5 74.4) (width 0.5) (layer "F.Cu") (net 2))
 (segment (start 125.77 93.16) (end 122.52 93.16) (width 0.5) (layer "F.Cu") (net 2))
 (segment (start 143.5 74.4) (end 147 77.9) (width 0.5) (layer "F.Cu") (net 2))
 (segment (start 117 89.48) (end 117 77.9) (width 0.5) (layer "F.Cu") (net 2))
 (segment (start 138 108) (end 147 108) (width 0.5) (layer "F.Cu") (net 2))
 (segment (start 147.9 97.6) (end 147.9 88.1) (width 0.5) (layer "F.Cu") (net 2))
 (segment (start 148 78.9) (end 147 77.9) (width 0.5) (layer "F.Cu") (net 2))
 (segment (start 129.74 89.18) (end 129.74 86.26) (width 0.5) (layer "F.Cu") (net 2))
 (via (at 125.77 93.16) (size 0.8) (drill 0.4) (layers "F.Cu" "B.Cu") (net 2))
 (segment (start 125.77 93.15) (end 125.77 93.16) (width 0.5) (layer "B.Cu") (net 2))
 (segment (start 129.74 89.18) (end 125.77 93.15) (width 0.5) (layer "B.Cu") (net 2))
 (segment (start 145.46 88) (end 142.08 88) (width 0.5) (layer "F.Cu") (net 9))
 (segment (start 142.08 88) (end 140 90.08) (width 0.5) (layer "F.Cu") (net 9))
 (segment (start 145.36 97.6) (end 141.68 97.6) (width 0.5) (layer "F.Cu") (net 11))
 (segment (start 141.68 97.6) (end 140 95.92) (width 0.5) (layer "F.Cu") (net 11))
 (segment (start 134.82 92.05) (end 134.82 96.8) (width 0.5) (layer "F.Cu") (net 6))
 (segment (start 140 79.92) (end 140 86.81) (width 0.5) (layer "F.Cu") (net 6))
 (segment (start 140 86.81) (end 134.79 92.02) (width 0.5) (layer "F.Cu") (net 6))
 (segment (start 134.79 92.02) (end 134.82 92.05) (width 0.5) (layer "F.Cu") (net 6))
 (segment (start 135.83 84.09) (end 140 79.92) (width 0.5) (layer "B.Cu") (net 6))
 (segment (start 126.51 84.09) (end 135.83 84.09) (width 0.5) (layer "B.Cu") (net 6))
 (segment (start 121.6 89) (end 126.51 84.09) (width 0.5) (layer "B.Cu") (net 6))
 (segment (start 136.08 78) (end 136.08 87.92) (width 0.5) (layer "F.Cu") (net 7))
 (segment (start 132.46 91.54) (end 121.6 91.54) (width 0.5) (layer "F.Cu") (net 7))
 (segment (start 134.82 89.18) (end 132.46 91.54) (width 0.5) (layer "F.Cu") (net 7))
 (segment (start 136.08 87.92) (end 134.82 89.18) (width 0.5) (layer "F.Cu") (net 7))
 (segment (start 127.91 94.97) (end 123.25 94.97) (width 0.5) (layer "F.Cu") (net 4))
 (segment (start 123.25 94.97) (end 121.6 96.62) (width 0.5) (layer "F.Cu") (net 4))
 (segment (start 129.74 96.8) (end 127.91 94.97) (width 0.5) (layer "F.Cu") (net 4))
 (segment (start 126 103.56) (end 121.6 99.16) (width 0.5) (layer "F.Cu") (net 8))
 (segment (start 126 108) (end 126 103.56) (width 0.5) (layer "F.Cu") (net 8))
 (segment (start 124.46 91.92) (end 127.2 89.18) (width 0.5) (layer "B.Cu") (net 8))
 (segment (start 121.6 99.16) (end 124.46 96.3) (width 0.5) (layer "B.Cu") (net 8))
 (segment (start 124.46 96.3) (end 124.46 91.92) (width 0.5) (layer "B.Cu") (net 8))
 (segment (start 138.36 106.08) (end 132.28 100) (width 0.5) (layer "F.Cu") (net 5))
 (segment (start 132.28 100) (end 132.28 96.8) (width 0.5) (layer "F.Cu") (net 5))
 (segment (start 140 106.08) (end 138.36 106.08) (width 0.5) (layer "F.Cu") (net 5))
 (segment (start 131.5 108) (end 127.75 104.25) (width 0.5) (layer "F.Cu") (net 3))
 (segment (start 136.16 108) (end 131.5 108) (width 0.5) (layer "F.Cu") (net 3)))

